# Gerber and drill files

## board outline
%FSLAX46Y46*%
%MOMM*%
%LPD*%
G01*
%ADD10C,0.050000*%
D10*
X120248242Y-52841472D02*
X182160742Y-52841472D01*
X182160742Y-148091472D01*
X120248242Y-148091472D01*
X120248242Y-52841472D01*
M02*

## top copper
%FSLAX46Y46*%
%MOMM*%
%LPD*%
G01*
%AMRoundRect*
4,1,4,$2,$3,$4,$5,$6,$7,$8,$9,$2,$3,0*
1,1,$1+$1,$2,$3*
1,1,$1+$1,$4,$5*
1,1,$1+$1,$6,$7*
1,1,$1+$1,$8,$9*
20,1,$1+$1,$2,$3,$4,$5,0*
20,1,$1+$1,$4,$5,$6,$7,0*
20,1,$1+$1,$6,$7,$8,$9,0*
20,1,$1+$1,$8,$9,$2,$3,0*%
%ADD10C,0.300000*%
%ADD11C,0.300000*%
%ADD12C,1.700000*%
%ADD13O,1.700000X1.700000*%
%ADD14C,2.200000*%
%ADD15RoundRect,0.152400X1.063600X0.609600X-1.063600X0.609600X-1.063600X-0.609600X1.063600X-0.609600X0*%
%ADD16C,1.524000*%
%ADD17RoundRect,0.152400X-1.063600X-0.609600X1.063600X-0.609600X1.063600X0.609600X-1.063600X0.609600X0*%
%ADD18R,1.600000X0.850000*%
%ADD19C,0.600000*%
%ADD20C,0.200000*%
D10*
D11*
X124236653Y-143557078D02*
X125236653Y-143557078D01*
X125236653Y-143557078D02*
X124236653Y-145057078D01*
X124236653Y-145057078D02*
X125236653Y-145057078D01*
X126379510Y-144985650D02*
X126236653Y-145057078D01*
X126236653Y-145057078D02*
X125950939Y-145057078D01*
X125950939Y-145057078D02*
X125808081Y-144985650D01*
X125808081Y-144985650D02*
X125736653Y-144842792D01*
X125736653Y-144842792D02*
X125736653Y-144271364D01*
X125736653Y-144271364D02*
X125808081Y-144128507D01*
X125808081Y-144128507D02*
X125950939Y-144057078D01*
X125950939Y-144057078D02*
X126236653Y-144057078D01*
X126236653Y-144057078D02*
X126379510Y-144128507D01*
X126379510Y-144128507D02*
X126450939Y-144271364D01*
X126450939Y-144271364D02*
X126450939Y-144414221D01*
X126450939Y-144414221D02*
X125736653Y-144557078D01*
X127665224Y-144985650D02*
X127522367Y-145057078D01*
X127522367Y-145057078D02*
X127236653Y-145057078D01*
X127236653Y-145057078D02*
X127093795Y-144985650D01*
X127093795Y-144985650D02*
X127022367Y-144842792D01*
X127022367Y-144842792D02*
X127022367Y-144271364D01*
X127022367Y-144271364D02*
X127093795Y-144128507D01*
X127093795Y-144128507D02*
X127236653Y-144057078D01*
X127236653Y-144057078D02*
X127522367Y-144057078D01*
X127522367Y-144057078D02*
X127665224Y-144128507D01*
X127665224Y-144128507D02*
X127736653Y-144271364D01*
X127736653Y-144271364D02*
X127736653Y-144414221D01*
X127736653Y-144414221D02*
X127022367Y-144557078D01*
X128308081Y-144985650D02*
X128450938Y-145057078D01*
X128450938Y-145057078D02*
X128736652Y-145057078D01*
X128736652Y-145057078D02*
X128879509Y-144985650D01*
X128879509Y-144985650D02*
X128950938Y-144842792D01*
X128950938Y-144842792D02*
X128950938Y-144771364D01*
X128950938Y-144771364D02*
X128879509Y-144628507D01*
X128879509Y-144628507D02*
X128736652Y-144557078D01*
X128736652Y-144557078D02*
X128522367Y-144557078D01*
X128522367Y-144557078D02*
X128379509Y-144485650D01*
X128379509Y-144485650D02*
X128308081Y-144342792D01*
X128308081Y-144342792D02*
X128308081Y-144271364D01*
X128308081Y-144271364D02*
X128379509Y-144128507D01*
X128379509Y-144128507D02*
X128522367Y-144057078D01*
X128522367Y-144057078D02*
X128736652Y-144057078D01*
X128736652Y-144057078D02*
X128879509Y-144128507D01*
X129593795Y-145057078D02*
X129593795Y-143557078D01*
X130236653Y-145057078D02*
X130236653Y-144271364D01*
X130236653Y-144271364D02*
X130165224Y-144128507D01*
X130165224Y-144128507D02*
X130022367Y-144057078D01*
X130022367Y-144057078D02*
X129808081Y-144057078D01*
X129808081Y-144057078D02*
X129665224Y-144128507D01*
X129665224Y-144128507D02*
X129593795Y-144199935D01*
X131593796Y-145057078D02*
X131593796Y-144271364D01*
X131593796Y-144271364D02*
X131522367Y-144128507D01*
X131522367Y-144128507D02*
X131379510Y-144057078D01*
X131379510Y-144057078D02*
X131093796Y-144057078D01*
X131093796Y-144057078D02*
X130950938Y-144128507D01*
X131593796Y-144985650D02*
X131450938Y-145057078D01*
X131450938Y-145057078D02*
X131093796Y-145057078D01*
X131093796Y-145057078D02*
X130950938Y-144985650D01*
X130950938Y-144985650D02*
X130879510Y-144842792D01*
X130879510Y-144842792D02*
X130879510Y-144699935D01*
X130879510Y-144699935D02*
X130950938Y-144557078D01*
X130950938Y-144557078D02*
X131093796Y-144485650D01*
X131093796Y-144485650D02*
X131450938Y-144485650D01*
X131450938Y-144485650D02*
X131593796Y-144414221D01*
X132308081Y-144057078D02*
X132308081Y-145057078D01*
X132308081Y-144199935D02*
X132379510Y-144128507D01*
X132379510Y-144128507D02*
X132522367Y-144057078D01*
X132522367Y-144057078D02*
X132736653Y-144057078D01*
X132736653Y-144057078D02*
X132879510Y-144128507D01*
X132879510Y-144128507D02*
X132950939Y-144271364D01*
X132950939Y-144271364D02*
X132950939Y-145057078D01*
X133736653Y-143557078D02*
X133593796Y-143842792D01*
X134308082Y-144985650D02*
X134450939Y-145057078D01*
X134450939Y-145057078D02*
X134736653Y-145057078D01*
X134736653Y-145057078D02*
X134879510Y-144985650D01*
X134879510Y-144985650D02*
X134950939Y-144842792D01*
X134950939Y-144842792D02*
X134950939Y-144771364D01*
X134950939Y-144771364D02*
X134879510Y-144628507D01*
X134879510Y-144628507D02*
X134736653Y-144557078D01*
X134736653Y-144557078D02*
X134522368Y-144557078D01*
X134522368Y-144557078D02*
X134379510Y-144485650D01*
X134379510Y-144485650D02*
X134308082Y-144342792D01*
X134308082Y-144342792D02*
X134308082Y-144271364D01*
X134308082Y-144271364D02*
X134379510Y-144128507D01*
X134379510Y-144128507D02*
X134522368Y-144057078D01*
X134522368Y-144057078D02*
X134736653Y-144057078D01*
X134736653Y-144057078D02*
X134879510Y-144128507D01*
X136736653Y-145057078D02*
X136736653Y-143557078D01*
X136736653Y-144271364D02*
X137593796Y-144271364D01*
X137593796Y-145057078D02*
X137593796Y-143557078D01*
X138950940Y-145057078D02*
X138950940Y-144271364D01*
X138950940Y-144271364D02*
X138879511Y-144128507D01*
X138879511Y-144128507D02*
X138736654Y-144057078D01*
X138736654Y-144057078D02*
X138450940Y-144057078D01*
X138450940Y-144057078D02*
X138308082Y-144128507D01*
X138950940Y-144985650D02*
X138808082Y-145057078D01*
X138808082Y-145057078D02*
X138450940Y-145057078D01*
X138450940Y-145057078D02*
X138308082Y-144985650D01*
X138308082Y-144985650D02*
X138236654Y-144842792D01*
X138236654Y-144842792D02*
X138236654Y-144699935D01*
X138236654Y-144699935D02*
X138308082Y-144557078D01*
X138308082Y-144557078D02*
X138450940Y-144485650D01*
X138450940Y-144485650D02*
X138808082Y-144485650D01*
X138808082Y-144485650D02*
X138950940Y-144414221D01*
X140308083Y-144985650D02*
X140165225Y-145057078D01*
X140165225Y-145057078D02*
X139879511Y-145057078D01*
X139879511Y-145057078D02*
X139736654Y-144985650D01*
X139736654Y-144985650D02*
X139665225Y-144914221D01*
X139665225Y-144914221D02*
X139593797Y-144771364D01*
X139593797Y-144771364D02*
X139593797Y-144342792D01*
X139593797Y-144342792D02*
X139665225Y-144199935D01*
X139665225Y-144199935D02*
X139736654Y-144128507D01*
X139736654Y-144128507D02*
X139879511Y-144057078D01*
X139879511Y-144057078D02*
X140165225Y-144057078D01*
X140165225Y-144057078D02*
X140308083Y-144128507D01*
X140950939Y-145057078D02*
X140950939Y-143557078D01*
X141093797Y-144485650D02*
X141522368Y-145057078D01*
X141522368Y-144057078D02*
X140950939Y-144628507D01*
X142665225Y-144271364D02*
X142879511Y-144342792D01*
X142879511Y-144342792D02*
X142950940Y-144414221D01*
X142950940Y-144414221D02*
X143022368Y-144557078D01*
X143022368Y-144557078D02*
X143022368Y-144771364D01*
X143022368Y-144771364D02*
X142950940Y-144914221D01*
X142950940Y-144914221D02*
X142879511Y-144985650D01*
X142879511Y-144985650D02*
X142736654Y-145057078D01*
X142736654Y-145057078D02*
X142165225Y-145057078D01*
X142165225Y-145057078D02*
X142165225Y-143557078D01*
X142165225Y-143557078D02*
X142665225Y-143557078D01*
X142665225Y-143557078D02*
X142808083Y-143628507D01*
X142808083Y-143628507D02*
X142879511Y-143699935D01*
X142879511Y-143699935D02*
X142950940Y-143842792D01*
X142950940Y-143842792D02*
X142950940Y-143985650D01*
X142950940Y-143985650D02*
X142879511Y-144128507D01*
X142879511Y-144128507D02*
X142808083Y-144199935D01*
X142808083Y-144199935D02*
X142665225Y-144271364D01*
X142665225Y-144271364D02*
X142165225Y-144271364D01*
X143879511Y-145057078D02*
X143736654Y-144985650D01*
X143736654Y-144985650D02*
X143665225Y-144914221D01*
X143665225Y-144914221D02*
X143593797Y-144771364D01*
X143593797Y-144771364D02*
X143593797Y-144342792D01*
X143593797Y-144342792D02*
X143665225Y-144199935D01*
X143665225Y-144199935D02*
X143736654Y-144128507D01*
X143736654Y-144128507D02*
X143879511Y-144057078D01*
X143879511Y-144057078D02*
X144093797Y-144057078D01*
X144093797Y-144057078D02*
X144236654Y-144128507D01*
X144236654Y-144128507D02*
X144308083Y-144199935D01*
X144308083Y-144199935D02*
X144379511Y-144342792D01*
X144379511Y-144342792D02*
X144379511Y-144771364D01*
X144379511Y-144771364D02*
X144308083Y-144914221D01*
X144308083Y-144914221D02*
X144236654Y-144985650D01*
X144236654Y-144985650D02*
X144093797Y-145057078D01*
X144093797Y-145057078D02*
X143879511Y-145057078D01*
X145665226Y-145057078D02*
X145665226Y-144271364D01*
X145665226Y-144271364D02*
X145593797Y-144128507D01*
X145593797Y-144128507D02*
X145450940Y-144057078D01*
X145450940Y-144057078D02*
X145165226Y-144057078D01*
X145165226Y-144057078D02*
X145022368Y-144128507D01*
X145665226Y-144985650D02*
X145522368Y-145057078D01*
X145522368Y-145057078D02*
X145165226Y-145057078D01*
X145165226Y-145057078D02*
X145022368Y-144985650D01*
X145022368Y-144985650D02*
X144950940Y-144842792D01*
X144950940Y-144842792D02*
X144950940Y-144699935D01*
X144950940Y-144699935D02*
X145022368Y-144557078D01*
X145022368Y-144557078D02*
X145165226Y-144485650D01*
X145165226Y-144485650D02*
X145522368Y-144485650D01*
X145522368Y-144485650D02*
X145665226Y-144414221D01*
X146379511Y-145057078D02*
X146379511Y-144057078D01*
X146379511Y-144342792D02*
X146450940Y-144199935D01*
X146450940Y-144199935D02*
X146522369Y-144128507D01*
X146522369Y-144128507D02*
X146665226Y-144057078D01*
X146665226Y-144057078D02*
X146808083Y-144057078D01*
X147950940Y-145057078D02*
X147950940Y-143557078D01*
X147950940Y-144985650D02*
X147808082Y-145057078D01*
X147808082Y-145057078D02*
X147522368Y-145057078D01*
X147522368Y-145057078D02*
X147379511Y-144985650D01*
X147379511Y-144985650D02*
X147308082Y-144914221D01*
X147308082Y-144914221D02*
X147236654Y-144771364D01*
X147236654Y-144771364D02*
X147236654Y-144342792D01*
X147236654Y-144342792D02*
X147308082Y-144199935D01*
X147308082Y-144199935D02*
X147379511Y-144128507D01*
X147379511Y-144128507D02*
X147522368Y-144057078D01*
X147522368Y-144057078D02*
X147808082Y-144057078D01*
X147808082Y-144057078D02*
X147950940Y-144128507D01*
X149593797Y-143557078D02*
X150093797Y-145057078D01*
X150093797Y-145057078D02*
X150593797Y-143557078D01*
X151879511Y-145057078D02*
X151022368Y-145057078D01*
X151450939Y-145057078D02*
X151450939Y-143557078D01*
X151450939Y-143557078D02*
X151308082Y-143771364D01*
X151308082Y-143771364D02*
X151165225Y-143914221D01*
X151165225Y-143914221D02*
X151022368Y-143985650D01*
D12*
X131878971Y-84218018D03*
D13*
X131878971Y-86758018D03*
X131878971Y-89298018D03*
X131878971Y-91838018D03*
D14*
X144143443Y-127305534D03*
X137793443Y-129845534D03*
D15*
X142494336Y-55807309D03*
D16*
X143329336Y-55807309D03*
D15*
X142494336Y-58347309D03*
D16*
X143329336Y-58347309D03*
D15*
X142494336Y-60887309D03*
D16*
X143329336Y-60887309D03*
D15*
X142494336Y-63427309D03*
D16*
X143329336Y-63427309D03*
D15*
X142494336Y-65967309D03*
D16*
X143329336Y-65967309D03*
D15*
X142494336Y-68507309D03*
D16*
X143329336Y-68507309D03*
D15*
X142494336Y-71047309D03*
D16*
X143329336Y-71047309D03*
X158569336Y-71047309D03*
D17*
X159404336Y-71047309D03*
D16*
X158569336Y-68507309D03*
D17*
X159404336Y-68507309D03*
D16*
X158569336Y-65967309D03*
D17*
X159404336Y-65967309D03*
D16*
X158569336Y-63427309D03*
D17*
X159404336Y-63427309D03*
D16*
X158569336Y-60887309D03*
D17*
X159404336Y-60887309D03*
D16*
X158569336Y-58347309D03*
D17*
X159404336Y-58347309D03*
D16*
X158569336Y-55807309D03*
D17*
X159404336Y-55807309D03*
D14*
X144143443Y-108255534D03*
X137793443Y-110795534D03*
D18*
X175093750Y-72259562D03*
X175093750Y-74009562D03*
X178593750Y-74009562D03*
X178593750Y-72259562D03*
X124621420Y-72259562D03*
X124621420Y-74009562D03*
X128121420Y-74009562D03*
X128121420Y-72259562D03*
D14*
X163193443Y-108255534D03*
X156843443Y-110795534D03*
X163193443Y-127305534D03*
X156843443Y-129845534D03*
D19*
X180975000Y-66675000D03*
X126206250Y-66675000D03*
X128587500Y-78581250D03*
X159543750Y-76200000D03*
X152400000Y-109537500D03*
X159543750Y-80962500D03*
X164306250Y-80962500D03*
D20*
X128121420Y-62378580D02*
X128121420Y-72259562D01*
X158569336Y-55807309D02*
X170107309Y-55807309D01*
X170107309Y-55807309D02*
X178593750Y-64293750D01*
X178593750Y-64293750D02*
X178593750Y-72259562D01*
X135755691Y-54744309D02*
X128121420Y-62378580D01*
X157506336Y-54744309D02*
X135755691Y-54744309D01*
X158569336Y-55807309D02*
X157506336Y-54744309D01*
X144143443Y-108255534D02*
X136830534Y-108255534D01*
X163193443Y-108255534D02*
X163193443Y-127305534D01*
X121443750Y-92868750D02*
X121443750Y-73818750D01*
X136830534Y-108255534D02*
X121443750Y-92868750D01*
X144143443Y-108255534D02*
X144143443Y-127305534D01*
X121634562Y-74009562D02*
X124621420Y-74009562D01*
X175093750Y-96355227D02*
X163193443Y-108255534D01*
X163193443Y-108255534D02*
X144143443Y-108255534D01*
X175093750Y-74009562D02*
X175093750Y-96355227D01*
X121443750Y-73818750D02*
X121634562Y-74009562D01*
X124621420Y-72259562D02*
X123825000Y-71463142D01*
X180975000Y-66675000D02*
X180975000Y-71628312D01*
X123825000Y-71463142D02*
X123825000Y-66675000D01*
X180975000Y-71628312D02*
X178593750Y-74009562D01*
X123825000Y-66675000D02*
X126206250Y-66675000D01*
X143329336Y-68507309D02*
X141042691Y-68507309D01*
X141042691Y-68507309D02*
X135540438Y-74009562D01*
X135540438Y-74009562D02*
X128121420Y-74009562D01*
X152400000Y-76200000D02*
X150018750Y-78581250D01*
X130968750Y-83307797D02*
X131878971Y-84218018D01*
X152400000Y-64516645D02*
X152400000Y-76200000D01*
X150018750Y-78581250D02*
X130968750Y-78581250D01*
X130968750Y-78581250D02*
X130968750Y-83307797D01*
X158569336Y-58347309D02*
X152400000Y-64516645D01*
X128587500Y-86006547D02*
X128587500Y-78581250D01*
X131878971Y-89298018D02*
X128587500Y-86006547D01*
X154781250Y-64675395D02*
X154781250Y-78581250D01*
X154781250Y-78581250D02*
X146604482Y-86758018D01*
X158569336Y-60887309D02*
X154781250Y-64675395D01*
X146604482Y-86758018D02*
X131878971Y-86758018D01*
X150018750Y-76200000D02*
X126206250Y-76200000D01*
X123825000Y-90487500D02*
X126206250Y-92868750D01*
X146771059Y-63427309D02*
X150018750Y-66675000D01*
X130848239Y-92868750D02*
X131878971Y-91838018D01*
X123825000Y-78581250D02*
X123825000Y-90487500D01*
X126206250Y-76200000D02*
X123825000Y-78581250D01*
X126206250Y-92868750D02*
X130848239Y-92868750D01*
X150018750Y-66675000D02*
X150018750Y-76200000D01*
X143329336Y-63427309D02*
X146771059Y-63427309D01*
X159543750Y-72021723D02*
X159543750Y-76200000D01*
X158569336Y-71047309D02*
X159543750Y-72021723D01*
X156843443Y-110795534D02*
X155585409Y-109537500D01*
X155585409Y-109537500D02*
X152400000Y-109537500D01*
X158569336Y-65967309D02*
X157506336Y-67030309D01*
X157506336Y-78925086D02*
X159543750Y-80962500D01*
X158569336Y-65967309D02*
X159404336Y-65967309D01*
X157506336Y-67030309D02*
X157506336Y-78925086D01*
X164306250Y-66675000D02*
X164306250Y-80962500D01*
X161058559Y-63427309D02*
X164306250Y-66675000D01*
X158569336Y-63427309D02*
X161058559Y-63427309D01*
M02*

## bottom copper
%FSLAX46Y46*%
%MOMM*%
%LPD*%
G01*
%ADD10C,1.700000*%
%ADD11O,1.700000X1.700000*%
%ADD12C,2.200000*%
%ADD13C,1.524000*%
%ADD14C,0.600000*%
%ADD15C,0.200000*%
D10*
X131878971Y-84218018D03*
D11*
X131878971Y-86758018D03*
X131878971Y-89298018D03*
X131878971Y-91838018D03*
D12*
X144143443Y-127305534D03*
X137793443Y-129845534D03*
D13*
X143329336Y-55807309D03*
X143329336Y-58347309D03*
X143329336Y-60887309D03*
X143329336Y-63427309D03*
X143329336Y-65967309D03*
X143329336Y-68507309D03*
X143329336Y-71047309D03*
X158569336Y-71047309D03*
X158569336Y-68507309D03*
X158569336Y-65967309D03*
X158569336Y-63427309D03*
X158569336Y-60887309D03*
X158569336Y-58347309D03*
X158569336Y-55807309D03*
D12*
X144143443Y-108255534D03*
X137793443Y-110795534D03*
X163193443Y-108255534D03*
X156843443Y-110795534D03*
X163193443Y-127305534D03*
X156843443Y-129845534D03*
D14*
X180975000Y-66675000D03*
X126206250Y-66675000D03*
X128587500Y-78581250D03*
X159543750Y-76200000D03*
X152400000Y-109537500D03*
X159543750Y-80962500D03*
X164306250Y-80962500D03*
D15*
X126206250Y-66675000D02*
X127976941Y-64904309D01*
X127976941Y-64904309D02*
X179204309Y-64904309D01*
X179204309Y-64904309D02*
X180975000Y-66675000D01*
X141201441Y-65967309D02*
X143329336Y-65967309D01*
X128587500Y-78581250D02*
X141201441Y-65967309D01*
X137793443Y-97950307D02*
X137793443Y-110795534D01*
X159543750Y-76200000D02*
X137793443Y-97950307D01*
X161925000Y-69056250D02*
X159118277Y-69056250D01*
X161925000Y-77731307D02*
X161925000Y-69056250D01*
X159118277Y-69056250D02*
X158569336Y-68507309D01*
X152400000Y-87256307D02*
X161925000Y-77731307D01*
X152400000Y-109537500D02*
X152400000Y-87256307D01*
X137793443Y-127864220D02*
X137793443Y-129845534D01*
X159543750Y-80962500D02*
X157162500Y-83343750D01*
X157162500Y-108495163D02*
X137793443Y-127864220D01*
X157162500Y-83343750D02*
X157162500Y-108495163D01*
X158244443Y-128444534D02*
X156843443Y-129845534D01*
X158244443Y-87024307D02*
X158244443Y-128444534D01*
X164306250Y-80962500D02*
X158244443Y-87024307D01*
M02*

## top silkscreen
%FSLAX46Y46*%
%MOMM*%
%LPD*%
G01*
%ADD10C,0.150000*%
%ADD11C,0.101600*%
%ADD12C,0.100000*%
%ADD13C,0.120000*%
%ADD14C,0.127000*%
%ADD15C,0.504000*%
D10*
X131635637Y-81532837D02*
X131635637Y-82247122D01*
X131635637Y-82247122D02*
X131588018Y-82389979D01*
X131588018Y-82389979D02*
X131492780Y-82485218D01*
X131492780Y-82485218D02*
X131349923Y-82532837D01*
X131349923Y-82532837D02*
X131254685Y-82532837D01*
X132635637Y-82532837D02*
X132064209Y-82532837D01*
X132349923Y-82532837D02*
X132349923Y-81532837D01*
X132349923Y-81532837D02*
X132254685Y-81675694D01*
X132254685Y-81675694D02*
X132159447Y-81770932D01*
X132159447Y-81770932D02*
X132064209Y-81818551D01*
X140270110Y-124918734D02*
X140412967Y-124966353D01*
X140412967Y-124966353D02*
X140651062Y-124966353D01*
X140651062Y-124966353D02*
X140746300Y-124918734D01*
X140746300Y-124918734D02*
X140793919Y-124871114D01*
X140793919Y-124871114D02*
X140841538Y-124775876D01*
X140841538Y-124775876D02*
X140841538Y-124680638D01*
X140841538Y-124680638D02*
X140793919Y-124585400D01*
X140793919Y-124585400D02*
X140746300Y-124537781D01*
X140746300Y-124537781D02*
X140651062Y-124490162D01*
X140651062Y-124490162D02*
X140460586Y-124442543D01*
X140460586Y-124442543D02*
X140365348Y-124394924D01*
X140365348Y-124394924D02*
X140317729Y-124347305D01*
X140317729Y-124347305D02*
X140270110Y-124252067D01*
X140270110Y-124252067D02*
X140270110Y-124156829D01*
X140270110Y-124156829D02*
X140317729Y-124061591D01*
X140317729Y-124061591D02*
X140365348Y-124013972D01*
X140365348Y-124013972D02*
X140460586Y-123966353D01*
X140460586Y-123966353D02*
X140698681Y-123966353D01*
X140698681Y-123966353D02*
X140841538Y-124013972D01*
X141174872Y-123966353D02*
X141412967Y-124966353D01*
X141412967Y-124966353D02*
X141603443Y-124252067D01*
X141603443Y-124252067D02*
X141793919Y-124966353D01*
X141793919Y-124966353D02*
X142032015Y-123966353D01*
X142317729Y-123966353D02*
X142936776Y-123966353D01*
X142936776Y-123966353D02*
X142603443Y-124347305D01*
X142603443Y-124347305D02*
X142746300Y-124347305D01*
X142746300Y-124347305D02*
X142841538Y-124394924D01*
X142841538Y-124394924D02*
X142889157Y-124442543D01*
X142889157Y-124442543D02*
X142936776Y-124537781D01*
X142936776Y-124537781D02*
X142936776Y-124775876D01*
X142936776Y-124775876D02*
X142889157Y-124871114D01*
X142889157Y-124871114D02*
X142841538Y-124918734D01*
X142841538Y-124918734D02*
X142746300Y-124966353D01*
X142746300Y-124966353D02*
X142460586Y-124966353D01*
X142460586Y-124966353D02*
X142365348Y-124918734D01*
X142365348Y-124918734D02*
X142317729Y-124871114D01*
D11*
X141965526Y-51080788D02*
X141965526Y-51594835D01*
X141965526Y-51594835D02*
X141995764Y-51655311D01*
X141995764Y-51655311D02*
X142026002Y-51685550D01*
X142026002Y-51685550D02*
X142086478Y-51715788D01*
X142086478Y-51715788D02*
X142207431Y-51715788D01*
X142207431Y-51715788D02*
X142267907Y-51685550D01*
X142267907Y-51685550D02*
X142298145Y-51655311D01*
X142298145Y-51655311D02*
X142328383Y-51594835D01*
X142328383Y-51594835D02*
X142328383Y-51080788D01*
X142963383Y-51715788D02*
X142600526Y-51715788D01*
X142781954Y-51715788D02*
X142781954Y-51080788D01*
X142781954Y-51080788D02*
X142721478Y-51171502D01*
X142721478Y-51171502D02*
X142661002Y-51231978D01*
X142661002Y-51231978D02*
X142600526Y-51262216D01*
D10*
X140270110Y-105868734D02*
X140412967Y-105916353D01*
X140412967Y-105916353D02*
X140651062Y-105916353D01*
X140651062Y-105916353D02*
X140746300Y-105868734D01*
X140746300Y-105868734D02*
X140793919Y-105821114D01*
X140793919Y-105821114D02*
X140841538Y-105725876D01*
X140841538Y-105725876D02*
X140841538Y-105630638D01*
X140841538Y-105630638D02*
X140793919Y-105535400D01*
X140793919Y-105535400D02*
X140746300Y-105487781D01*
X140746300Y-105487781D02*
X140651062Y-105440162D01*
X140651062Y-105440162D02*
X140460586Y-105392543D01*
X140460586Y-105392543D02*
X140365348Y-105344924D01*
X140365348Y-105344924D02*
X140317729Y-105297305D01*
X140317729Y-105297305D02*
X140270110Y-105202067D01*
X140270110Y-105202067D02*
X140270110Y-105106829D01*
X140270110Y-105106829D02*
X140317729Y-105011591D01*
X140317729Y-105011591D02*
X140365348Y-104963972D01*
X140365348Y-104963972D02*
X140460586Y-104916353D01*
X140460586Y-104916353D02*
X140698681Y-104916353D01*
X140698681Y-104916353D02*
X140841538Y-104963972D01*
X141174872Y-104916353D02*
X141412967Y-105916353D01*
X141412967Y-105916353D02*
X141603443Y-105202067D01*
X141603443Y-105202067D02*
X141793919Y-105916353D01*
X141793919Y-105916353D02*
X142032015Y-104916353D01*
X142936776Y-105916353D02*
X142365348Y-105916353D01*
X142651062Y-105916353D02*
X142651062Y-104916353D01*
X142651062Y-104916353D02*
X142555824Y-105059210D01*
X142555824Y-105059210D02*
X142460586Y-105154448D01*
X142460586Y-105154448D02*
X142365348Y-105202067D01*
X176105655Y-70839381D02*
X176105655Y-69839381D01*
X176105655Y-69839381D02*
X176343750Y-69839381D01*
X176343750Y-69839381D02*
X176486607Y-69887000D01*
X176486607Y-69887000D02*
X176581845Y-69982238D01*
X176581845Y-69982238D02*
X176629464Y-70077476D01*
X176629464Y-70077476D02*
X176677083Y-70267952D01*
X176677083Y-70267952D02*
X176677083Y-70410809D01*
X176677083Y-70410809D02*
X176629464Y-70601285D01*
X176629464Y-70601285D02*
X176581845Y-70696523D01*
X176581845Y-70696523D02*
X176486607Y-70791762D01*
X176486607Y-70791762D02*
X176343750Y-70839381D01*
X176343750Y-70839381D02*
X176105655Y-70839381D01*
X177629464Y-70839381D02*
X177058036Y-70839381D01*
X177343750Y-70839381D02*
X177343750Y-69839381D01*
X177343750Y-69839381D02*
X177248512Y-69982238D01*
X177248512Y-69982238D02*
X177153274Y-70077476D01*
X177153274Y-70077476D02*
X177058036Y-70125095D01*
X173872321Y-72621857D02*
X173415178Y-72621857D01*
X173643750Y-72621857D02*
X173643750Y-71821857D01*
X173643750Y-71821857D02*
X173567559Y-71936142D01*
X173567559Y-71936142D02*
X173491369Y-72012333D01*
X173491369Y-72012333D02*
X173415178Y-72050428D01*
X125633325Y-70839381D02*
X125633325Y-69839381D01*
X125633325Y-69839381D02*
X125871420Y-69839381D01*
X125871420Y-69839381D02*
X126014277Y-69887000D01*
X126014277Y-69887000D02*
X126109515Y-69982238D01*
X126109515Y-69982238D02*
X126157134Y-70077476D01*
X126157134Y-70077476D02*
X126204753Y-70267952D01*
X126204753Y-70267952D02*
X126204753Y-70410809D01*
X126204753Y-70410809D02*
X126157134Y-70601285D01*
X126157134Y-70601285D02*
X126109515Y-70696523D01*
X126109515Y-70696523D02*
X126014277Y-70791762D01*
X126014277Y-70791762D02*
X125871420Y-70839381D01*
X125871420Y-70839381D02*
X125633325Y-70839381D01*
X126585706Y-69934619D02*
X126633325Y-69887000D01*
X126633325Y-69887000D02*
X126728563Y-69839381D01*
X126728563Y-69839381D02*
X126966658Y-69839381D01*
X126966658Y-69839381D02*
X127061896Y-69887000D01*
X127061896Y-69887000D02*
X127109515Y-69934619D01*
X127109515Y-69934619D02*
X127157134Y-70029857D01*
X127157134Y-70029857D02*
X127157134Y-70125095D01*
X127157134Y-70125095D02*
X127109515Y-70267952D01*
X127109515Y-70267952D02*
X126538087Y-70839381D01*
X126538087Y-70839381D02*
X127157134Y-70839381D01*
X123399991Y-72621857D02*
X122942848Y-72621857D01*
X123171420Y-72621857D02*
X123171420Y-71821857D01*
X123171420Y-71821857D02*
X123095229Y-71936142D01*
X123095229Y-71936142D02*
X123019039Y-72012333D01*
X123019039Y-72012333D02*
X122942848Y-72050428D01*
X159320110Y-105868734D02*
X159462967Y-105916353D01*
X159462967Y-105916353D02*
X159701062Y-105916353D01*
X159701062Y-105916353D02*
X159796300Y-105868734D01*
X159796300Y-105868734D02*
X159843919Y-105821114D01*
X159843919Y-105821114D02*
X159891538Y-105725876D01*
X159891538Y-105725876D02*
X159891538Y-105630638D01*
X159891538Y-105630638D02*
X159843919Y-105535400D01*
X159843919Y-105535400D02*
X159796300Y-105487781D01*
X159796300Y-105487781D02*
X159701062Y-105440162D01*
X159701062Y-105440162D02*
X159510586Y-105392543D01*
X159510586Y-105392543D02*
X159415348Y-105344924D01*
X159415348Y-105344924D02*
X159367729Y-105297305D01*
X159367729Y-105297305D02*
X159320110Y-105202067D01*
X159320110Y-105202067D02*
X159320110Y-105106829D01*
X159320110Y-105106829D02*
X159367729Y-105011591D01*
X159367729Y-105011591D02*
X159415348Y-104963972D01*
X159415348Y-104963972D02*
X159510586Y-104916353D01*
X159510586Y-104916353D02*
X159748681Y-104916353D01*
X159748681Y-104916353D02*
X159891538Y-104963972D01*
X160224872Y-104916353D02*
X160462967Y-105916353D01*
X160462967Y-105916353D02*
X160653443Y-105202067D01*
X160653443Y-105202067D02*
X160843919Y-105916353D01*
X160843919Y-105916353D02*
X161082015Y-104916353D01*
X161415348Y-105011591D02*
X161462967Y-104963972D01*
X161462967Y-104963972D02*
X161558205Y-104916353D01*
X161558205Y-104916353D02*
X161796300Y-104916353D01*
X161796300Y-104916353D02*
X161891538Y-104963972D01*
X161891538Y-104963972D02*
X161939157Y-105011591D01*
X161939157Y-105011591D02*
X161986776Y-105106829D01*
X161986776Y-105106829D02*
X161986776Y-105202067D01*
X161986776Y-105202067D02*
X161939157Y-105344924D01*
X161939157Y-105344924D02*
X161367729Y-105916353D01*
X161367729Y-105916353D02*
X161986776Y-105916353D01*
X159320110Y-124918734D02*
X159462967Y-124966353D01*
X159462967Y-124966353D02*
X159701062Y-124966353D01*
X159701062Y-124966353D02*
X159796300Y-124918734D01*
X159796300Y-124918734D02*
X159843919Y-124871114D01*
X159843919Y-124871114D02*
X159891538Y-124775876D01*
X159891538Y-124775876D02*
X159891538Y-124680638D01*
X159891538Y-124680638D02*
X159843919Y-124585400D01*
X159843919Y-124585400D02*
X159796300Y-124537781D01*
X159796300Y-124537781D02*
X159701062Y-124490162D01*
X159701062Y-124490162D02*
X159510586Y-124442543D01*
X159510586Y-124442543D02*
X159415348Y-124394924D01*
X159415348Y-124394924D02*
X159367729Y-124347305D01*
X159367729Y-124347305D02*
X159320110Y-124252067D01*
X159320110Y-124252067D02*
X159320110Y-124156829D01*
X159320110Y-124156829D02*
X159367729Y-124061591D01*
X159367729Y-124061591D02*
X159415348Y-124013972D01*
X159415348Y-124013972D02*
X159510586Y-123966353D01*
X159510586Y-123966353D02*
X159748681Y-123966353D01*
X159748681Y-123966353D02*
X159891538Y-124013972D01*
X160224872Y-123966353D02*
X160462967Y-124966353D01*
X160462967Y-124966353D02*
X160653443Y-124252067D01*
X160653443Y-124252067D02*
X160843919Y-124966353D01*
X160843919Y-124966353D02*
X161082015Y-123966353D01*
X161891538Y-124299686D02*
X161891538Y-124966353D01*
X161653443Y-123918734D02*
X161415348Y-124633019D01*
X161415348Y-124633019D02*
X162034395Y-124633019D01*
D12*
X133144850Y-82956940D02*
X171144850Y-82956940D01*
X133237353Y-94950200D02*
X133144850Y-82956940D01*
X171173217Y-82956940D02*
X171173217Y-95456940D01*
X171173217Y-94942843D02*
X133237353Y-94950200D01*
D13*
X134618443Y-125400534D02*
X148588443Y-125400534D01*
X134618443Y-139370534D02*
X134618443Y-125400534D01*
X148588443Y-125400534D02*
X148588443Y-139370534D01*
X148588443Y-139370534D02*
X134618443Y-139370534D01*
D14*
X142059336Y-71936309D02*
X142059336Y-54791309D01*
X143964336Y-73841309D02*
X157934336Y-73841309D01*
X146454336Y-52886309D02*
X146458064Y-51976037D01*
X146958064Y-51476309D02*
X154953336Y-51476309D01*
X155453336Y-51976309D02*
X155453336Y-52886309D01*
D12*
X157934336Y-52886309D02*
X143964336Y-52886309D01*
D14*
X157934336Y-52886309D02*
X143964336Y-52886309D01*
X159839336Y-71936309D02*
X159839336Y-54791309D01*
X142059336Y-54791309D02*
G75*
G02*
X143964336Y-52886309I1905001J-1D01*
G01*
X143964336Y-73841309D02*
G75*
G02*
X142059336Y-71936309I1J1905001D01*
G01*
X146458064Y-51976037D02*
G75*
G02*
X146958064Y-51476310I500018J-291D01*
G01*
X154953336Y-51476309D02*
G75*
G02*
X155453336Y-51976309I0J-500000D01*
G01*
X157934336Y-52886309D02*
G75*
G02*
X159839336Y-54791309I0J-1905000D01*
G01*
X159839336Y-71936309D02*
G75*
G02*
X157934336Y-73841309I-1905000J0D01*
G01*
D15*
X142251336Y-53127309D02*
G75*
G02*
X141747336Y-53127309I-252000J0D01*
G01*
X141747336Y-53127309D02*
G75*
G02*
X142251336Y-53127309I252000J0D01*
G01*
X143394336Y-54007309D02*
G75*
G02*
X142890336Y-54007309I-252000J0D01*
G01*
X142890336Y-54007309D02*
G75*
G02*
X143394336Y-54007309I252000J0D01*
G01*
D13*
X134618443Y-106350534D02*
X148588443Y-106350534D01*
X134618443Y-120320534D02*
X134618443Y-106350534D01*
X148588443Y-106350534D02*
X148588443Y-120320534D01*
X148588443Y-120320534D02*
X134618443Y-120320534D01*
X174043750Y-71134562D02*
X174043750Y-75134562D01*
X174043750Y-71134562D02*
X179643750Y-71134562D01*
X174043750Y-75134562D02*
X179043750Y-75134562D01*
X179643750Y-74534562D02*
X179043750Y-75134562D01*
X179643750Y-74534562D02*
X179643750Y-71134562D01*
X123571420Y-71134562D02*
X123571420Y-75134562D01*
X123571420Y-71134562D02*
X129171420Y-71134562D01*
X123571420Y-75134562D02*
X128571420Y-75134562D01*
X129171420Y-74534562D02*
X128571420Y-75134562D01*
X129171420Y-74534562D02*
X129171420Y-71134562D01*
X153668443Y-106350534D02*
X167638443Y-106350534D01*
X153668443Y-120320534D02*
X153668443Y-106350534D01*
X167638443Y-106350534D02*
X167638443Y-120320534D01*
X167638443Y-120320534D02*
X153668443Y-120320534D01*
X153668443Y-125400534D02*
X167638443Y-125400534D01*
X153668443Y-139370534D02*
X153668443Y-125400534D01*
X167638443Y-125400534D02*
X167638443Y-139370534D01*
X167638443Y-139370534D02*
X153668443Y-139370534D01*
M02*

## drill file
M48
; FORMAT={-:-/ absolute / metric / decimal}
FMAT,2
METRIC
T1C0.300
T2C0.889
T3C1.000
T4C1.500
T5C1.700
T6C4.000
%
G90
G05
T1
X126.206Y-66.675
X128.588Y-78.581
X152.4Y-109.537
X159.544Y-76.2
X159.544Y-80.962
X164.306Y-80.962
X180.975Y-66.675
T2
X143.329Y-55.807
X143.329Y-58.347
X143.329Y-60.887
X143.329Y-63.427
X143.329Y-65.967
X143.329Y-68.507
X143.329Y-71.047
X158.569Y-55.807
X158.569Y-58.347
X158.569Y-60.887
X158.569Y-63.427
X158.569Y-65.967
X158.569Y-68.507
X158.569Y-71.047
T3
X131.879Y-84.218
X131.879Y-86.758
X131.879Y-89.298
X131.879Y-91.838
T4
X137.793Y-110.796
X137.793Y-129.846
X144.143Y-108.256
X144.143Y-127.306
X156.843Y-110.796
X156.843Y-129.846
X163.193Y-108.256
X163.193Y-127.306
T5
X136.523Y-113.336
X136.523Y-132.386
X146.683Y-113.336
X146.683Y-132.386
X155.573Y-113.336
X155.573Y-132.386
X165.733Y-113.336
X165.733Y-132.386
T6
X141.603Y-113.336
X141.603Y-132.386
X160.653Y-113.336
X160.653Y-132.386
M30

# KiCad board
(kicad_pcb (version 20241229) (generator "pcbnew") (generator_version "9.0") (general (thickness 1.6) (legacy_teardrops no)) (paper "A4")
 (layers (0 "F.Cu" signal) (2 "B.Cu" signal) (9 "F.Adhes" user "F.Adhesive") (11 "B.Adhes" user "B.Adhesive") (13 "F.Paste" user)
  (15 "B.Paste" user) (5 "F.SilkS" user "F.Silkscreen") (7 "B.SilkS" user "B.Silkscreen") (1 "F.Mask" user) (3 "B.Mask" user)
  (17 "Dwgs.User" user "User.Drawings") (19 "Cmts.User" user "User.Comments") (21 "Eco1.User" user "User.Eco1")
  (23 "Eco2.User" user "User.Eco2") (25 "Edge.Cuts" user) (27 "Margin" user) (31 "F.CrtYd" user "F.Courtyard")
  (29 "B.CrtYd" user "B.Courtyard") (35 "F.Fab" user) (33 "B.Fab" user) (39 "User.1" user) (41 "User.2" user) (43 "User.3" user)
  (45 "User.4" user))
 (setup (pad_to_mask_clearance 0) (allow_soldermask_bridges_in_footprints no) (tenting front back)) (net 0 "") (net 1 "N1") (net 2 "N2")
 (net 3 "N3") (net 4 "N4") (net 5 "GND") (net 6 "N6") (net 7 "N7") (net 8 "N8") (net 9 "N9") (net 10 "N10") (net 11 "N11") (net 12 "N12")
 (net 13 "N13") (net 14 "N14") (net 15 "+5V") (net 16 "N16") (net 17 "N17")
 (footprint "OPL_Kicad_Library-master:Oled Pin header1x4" (layer "F.Cu") (at 131.878971 84.218018)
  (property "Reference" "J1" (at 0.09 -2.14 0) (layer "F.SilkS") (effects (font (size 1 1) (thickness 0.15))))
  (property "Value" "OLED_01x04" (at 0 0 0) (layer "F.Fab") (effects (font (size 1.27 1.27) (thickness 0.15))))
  (fp_line (start 1.265879 -1.261078) (end 39.265879 -1.261078) (stroke (width 0.1) (type solid)) (layer "F.SilkS"))
  (fp_line (start 1.358382 10.732182) (end 1.265879 -1.261078) (stroke (width 0.1) (type default)) (layer "F.SilkS"))
  (fp_line (start 39.294246 -1.261078) (end 39.294246 11.238922) (stroke (width 0.1) (type solid)) (layer "F.SilkS"))
  (fp_line (start 39.294246 10.724825) (end 1.358382 10.732182) (stroke (width 0.1) (type default)) (layer "F.SilkS"))
  (pad "1" thru_hole circle (at 0 0) (size 1.7 1.7) (drill 1) (layers "*.Cu" "*.Mask") (remove_unused_layers no) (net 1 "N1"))
  (pad "2" thru_hole oval (at 0 2.54) (size 1.7 1.7) (drill 1) (layers "*.Cu" "*.Mask") (remove_unused_layers no) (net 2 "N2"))
  (pad "3" thru_hole oval (at 0 5.08) (size 1.7 1.7) (drill 1) (layers "*.Cu" "*.Mask") (remove_unused_layers no) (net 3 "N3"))
  (pad "4" thru_hole oval (at 0 7.62) (size 1.7 1.7) (drill 1) (layers "*.Cu" "*.Mask") (remove_unused_layers no) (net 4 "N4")))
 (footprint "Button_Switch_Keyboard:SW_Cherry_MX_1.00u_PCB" (layer "F.Cu") (at 144.143443 127.305534)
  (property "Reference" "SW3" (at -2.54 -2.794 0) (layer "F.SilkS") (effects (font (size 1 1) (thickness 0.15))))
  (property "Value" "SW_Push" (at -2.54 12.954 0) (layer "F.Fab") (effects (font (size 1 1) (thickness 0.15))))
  (fp_line (start -9.525 -1.905) (end 4.445 -1.905) (stroke (width 0.12) (type solid)) (layer "F.SilkS"))
  (fp_line (start -9.525 12.065) (end -9.525 -1.905) (stroke (width 0.12) (type solid)) (layer "F.SilkS"))
  (fp_line (start 4.445 -1.905) (end 4.445 12.065) (stroke (width 0.12) (type solid)) (layer "F.SilkS"))
  (fp_line (start 4.445 12.065) (end -9.525 12.065) (stroke (width 0.12) (type solid)) (layer "F.SilkS"))
  (pad "" np_thru_hole circle (at -7.62 5.08) (size 1.7 1.7) (drill 1.7) (layers "*.Cu" "*.Mask"))
  (pad "" np_thru_hole circle (at -2.54 5.08) (size 4 4) (drill 4) (layers "*.Cu" "*.Mask"))
  (pad "" np_thru_hole circle (at 2.54 5.08) (size 1.7 1.7) (drill 1.7) (layers "*.Cu" "*.Mask"))
  (pad "1" thru_hole circle (at 0 0) (size 2.2 2.2) (drill 1.5) (layers "*.Cu" "*.Mask") (remove_unused_layers no) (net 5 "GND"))
  (pad "2" thru_hole circle (at -6.35 2.54) (size 2.2 2.2) (drill 1.5) (layers "*.Cu" "*.Mask") (remove_unused_layers no) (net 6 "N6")))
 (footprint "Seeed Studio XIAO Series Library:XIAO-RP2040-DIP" (layer "F.Cu") (at 150.949336 63.427309)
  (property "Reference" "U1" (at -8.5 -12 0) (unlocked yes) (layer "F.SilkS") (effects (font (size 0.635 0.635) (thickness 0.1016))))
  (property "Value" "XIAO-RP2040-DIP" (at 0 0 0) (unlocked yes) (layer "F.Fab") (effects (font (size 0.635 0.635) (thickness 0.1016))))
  (fp_line (start -8.89 8.509) (end -8.89 -8.636) (stroke (width 0.127) (type solid)) (layer "F.SilkS"))
  (fp_line (start -6.985 10.414) (end 6.985 10.414) (stroke (width 0.127) (type solid)) (layer "F.SilkS"))
  (fp_line (start -4.495 -10.541) (end -4.491272 -11.451272) (stroke (width 0.127) (type solid)) (layer "F.SilkS"))
  (fp_line (start -3.991272 -11.951) (end 4.004 -11.951) (stroke (width 0.127) (type solid)) (layer "F.SilkS"))
  (fp_line (start 4.504 -11.451) (end 4.504 -10.541) (stroke (width 0.127) (type solid)) (layer "F.SilkS"))
  (fp_line (start 6.985 -10.541) (end -6.985 -10.541) (stroke (width 0.1) (type solid)) (layer "F.SilkS"))
  (fp_line (start 6.985 -10.541) (end -6.985 -10.541) (stroke (width 0.127) (type solid)) (layer "F.SilkS"))
  (fp_line (start 8.89 8.509) (end 8.89 -8.636) (stroke (width 0.127) (type solid)) (layer "F.SilkS"))
  (fp_arc (start -8.89 -8.636) (mid -8.332038 -9.983038) (end -6.985 -10.541) (stroke (width 0.127) (type solid)) (layer "F.SilkS"))
  (fp_arc (start -6.985 10.414) (mid -8.332038 9.856038) (end -8.89 8.509) (stroke (width 0.127) (type solid)) (layer "F.SilkS"))
  (fp_arc (start -4.491272 -11.451272) (mid -4.344728 -11.80464) (end -3.991272 -11.951) (stroke (width 0.127) (type default))
   (layer "F.SilkS"))
  (fp_arc (start 4.004 -11.951) (mid 4.357553 -11.804553) (end 4.504 -11.451) (stroke (width 0.127) (type default)) (layer "F.SilkS"))
  (fp_arc (start 6.985 -10.541) (mid 8.332038 -9.983038) (end 8.89 -8.636) (stroke (width 0.127) (type solid)) (layer "F.SilkS"))
  (fp_arc (start 8.89 8.509) (mid 8.332038 9.856038) (end 6.985 10.414) (stroke (width 0.127) (type solid)) (layer "F.SilkS"))
  (fp_circle (center -8.95 -10.3) (end -8.95 -10.554) (stroke (width 0.5) (type solid)) (fill yes) (layer "F.SilkS"))
  (fp_circle (center -7.807 -9.42) (end -7.807 -9.674) (stroke (width 0.5) (type solid)) (fill yes) (layer "F.SilkS"))
  (pad "1" smd roundrect (at -8.455 -7.62 180) (size 2.432 1.524) (layers "F.Cu" "F.Mask") (roundrect_rratio 0.1) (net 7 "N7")
   (thermal_bridge_angle 45))
  (pad "1" thru_hole circle (at -7.62 -7.62 180) (size 1.524 1.524) (drill 0.889) (layers "*.Cu" "*.Mask") (remove_unused_layers no)
   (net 7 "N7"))
  (pad "2" smd roundrect (at -8.455 -5.08 180) (size 2.432 1.524) (layers "F.Cu" "F.Mask") (roundrect_rratio 0.1) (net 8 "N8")
   (thermal_bridge_angle 45))
  (pad "2" thru_hole circle (at -7.62 -5.08 180) (size 1.524 1.524) (drill 0.889) (layers "*.Cu" "*.Mask") (remove_unused_layers no)
   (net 8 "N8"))
  (pad "3" smd roundrect (at -8.455 -2.54 180) (size 2.432 1.524) (layers "F.Cu" "F.Mask") (roundrect_rratio 0.1) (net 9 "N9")
   (thermal_bridge_angle 45))
  (pad "3" thru_hole circle (at -7.62 -2.54 180) (size 1.524 1.524) (drill 0.889) (layers "*.Cu" "*.Mask") (remove_unused_layers no)
   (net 9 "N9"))
  (pad "4" smd roundrect (at -8.455 0 180) (size 2.432 1.524) (layers "F.Cu" "F.Mask") (roundrect_rratio 0.1) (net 4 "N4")
   (thermal_bridge_angle 45))
  (pad "4" thru_hole circle (at -7.62 0 180) (size 1.524 1.524) (drill 0.889) (layers "*.Cu" "*.Mask") (remove_unused_layers no)
   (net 4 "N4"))
  (pad "5" smd roundrect (at -8.455 2.54 180) (size 2.432 1.524) (layers "F.Cu" "F.Mask") (roundrect_rratio 0.1) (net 3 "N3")
   (thermal_bridge_angle 45))
  (pad "5" thru_hole circle (at -7.62 2.54 180) (size 1.524 1.524) (drill 0.889) (layers "*.Cu" "*.Mask") (remove_unused_layers no)
   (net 3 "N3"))
  (pad "6" smd roundrect (at -8.455 5.08 180) (size 2.432 1.524) (layers "F.Cu" "F.Mask") (roundrect_rratio 0.1) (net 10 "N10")
   (thermal_bridge_angle 45))
  (pad "6" thru_hole circle (at -7.62 5.08 180) (size 1.524 1.524) (drill 0.889) (layers "*.Cu" "*.Mask") (remove_unused_layers no)
   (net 10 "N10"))
  (pad "7" smd roundrect (at -8.455 7.62 180) (size 2.432 1.524) (layers "F.Cu" "F.Mask") (roundrect_rratio 0.1) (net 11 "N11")
   (thermal_bridge_angle 45))
  (pad "7" thru_hole circle (at -7.62 7.62 180) (size 1.524 1.524) (drill 0.889) (layers "*.Cu" "*.Mask") (remove_unused_layers no)
   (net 11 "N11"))
  (pad "8" thru_hole circle (at 7.62 7.62) (size 1.524 1.524) (drill 0.889) (layers "*.Cu" "*.Mask") (remove_unused_layers no)
   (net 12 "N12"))
  (pad "8" smd roundrect (at 8.455 7.62) (size 2.432 1.524) (layers "F.Cu" "F.Mask") (roundrect_rratio 0.1) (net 12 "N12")
   (thermal_bridge_angle 45))
  (pad "9" thru_hole circle (at 7.62 5.08) (size 1.524 1.524) (drill 0.889) (layers "*.Cu" "*.Mask") (remove_unused_layers no)
   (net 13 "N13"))
  (pad "9" smd roundrect (at 8.455 5.08) (size 2.432 1.524) (layers "F.Cu" "F.Mask") (roundrect_rratio 0.1) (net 13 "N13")
   (thermal_bridge_angle 45))
  (pad "10" thru_hole circle (at 7.62 2.54) (size 1.524 1.524) (drill 0.889) (layers "*.Cu" "*.Mask") (remove_unused_layers no) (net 6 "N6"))
  (pad "10" smd roundrect (at 8.455 2.54) (size 2.432 1.524) (layers "F.Cu" "F.Mask") (roundrect_rratio 0.1) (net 6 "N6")
   (thermal_bridge_angle 45))
  (pad "11" thru_hole circle (at 7.62 0) (size 1.524 1.524) (drill 0.889) (layers "*.Cu" "*.Mask") (remove_unused_layers no) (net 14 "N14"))
  (pad "11" smd roundrect (at 8.455 0) (size 2.432 1.524) (layers "F.Cu" "F.Mask") (roundrect_rratio 0.1) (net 14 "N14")
   (thermal_bridge_angle 45))
  (pad "12" thru_hole circle (at 7.62 -2.54) (size 1.524 1.524) (drill 0.889) (layers "*.Cu" "*.Mask") (remove_unused_layers no)
   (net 2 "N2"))
  (pad "12" smd roundrect (at 8.455 -2.54) (size 2.432 1.524) (layers "F.Cu" "F.Mask") (roundrect_rratio 0.1) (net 2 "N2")
   (thermal_bridge_angle 45))
  (pad "13" thru_hole circle (at 7.62 -5.08) (size 1.524 1.524) (drill 0.889) (layers "*.Cu" "*.Mask") (remove_unused_layers no)
   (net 1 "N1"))
  (pad "13" smd roundrect (at 8.455 -5.08) (size 2.432 1.524) (layers "F.Cu" "F.Mask") (roundrect_rratio 0.1) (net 1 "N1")
   (thermal_bridge_angle 45))
  (pad "14" thru_hole circle (at 7.62 -7.62) (size 1.524 1.524) (drill 0.889) (layers "*.Cu" "*.Mask") (remove_unused_layers no)
   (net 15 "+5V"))
  (pad "14" smd roundrect (at 8.455 -7.62) (size 2.432 1.524) (layers "F.Cu" "F.Mask") (roundrect_rratio 0.1) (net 15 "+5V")
   (thermal_bridge_angle 45)))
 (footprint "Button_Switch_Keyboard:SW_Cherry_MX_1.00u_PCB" (layer "F.Cu") (at 144.143443 108.255534)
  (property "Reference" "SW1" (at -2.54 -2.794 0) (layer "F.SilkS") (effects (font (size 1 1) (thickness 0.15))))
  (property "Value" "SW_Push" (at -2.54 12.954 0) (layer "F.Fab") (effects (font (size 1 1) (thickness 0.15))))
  (fp_line (start -9.525 -1.905) (end 4.445 -1.905) (stroke (width 0.12) (type solid)) (layer "F.SilkS"))
  (fp_line (start -9.525 12.065) (end -9.525 -1.905) (stroke (width 0.12) (type solid)) (layer "F.SilkS"))
  (fp_line (start 4.445 -1.905) (end 4.445 12.065) (stroke (width 0.12) (type solid)) (layer "F.SilkS"))
  (fp_line (start 4.445 12.065) (end -9.525 12.065) (stroke (width 0.12) (type solid)) (layer "F.SilkS"))
  (pad "" np_thru_hole circle (at -7.62 5.08) (size 1.7 1.7) (drill 1.7) (layers "*.Cu" "*.Mask"))
  (pad "" np_thru_hole circle (at -2.54 5.08) (size 4 4) (drill 4) (layers "*.Cu" "*.Mask"))
  (pad "" np_thru_hole circle (at 2.54 5.08) (size 1.7 1.7) (drill 1.7) (layers "*.Cu" "*.Mask"))
  (pad "1" thru_hole circle (at 0 0) (size 2.2 2.2) (drill 1.5) (layers "*.Cu" "*.Mask") (remove_unused_layers no) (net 5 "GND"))
  (pad "2" thru_hole circle (at -6.35 2.54) (size 2.2 2.2) (drill 1.5) (layers "*.Cu" "*.Mask") (remove_unused_layers no) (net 12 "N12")))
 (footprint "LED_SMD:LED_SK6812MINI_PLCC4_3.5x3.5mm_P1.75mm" (layer "F.Cu") (at 176.84375 73.134562)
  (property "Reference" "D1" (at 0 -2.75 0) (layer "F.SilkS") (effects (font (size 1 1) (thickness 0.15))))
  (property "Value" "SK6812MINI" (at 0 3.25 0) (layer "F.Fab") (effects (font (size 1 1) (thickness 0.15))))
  (fp_line (start -2.8 -2) (end -2.8 2) (stroke (width 0.12) (type default)) (layer "F.SilkS"))
  (fp_line (start -2.8 -2) (end 2.8 -2) (stroke (width 0.12) (type solid)) (layer "F.SilkS"))
  (fp_line (start -2.8 2) (end 2.2 2) (stroke (width 0.12) (type solid)) (layer "F.SilkS"))
  (fp_line (start 2.8 1.4) (end 2.2 2) (stroke (width 0.12) (type default)) (layer "F.SilkS"))
  (fp_line (start 2.8 1.4) (end 2.8 -2) (stroke (width 0.12) (type solid)) (layer "F.SilkS"))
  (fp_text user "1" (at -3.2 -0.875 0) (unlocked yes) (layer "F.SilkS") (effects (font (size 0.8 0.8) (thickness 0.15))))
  (pad "1" smd rect (at -1.75 -0.875) (size 1.6 0.85) (layers "F.Cu" "F.Mask" "F.Paste") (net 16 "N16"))
  (pad "2" smd rect (at -1.75 0.875) (size 1.6 0.85) (layers "F.Cu" "F.Mask" "F.Paste") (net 5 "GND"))
  (pad "3" smd rect (at 1.75 0.875) (size 1.6 0.85) (layers "F.Cu" "F.Mask" "F.Paste") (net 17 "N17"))
  (pad "4" smd rect (at 1.75 -0.875) (size 1.6 0.85) (layers "F.Cu" "F.Mask" "F.Paste") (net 15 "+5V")))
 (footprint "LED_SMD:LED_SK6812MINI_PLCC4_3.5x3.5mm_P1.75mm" (layer "F.Cu") (at 126.37142 73.134562)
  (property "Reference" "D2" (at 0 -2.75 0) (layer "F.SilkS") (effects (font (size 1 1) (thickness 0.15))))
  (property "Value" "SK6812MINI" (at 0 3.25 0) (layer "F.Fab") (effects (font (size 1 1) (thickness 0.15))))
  (fp_line (start -2.8 -2) (end -2.8 2) (stroke (width 0.12) (type default)) (layer "F.SilkS"))
  (fp_line (start -2.8 -2) (end 2.8 -2) (stroke (width 0.12) (type solid)) (layer "F.SilkS"))
  (fp_line (start -2.8 2) (end 2.2 2) (stroke (width 0.12) (type solid)) (layer "F.SilkS"))
  (fp_line (start 2.8 1.4) (end 2.2 2) (stroke (width 0.12) (type default)) (layer "F.SilkS"))
  (fp_line (start 2.8 1.4) (end 2.8 -2) (stroke (width 0.12) (type solid)) (layer "F.SilkS"))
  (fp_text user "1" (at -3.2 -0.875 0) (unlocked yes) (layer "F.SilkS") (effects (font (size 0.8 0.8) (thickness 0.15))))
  (pad "1" smd rect (at -1.75 -0.875) (size 1.6 0.85) (layers "F.Cu" "F.Mask" "F.Paste") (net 17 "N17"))
  (pad "2" smd rect (at -1.75 0.875) (size 1.6 0.85) (layers "F.Cu" "F.Mask" "F.Paste") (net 5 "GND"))
  (pad "3" smd rect (at 1.75 0.875) (size 1.6 0.85) (layers "F.Cu" "F.Mask" "F.Paste") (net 10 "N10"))
  (pad "4" smd rect (at 1.75 -0.875) (size 1.6 0.85) (layers "F.Cu" "F.Mask" "F.Paste") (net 15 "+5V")))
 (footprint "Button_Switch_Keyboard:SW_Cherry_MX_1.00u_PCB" (layer "F.Cu") (at 163.193443 108.255534)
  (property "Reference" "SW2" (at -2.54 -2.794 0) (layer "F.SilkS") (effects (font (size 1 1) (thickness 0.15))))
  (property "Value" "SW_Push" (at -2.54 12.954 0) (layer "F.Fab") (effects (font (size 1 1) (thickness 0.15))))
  (fp_line (start -9.525 -1.905) (end 4.445 -1.905) (stroke (width 0.12) (type solid)) (layer "F.SilkS"))
  (fp_line (start -9.525 12.065) (end -9.525 -1.905) (stroke (width 0.12) (type solid)) (layer "F.SilkS"))
  (fp_line (start 4.445 -1.905) (end 4.445 12.065) (stroke (width 0.12) (type solid)) (layer "F.SilkS"))
  (fp_line (start 4.445 12.065) (end -9.525 12.065) (stroke (width 0.12) (type solid)) (layer "F.SilkS"))
  (pad "" np_thru_hole circle (at -7.62 5.08) (size 1.7 1.7) (drill 1.7) (layers "*.Cu" "*.Mask"))
  (pad "" np_thru_hole circle (at -2.54 5.08) (size 4 4) (drill 4) (layers "*.Cu" "*.Mask"))
  (pad "" np_thru_hole circle (at 2.54 5.08) (size 1.7 1.7) (drill 1.7) (layers "*.Cu" "*.Mask"))
  (pad "1" thru_hole circle (at 0 0) (size 2.2 2.2) (drill 1.5) (layers "*.Cu" "*.Mask") (remove_unused_layers no) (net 5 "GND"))
  (pad "2" thru_hole circle (at -6.35 2.54) (size 2.2 2.2) (drill 1.5) (layers "*.Cu" "*.Mask") (remove_unused_layers no) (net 13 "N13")))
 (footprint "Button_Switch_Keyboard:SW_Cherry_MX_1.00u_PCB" (layer "F.Cu") (at 163.193443 127.305534)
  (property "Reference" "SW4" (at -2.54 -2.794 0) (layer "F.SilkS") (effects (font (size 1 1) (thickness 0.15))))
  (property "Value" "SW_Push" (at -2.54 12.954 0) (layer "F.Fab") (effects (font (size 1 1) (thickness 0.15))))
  (fp_line (start -9.525 -1.905) (end 4.445 -1.905) (stroke (width 0.12) (type solid)) (layer "F.SilkS"))
  (fp_line (start -9.525 12.065) (end -9.525 -1.905) (stroke (width 0.12) (type solid)) (layer "F.SilkS"))
  (fp_line (start 4.445 -1.905) (end 4.445 12.065) (stroke (width 0.12) (type solid)) (layer "F.SilkS"))
  (fp_line (start 4.445 12.065) (end -9.525 12.065) (stroke (width 0.12) (type solid)) (layer "F.SilkS"))
  (pad "" np_thru_hole circle (at -7.62 5.08) (size 1.7 1.7) (drill 1.7) (layers "*.Cu" "*.Mask"))
  (pad "" np_thru_hole circle (at -2.54 5.08) (size 4 4) (drill 4) (layers "*.Cu" "*.Mask"))
  (pad "" np_thru_hole circle (at 2.54 5.08) (size 1.7 1.7) (drill 1.7) (layers "*.Cu" "*.Mask"))
  (pad "1" thru_hole circle (at 0 0) (size 2.2 2.2) (drill 1.5) (layers "*.Cu" "*.Mask") (remove_unused_layers no) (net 5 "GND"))
  (pad "2" thru_hole circle (at -6.35 2.54) (size 2.2 2.2) (drill 1.5) (layers "*.Cu" "*.Mask") (remove_unused_layers no) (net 14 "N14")))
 (gr_rect (start 120.248242 52.841472) (end 182.160742 148.091472) (stroke (width 0.05) (type default)) (fill no) (layer "Edge.Cuts"))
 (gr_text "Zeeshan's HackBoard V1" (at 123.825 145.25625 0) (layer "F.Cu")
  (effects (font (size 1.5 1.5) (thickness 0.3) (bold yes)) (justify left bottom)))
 (segment (start 128.12142 62.37858) (end 128.12142 72.259562) (width 0.2) (layer "F.Cu") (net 15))
 (segment (start 158.569336 55.807309) (end 170.107309 55.807309) (width 0.2) (layer "F.Cu") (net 15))
 (segment (start 170.107309 55.807309) (end 178.59375 64.29375) (width 0.2) (layer "F.Cu") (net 15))
 (segment (start 178.59375 64.29375) (end 178.59375 72.259562) (width 0.2) (layer "F.Cu") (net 15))
 (segment (start 135.755691 54.744309) (end 128.12142 62.37858) (width 0.2) (layer "F.Cu") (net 15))
 (segment (start 157.506336 54.744309) (end 135.755691 54.744309) (width 0.2) (layer "F.Cu") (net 15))
 (segment (start 158.569336 55.807309) (end 157.506336 54.744309) (width 0.2) (layer "F.Cu") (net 15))
 (segment (start 144.143443 108.255534) (end 136.830534 108.255534) (width 0.2) (layer "F.Cu") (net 5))
 (segment (start 163.193443 108.255534) (end 163.193443 127.305534) (width 0.2) (layer "F.Cu") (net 5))
 (segment (start 121.44375 92.86875) (end 121.44375 73.81875) (width 0.2) (layer "F.Cu") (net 5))
 (segment (start 136.830534 108.255534) (end 121.44375 92.86875) (width 0.2) (layer "F.Cu") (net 5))
 (segment (start 144.143443 108.255534) (end 144.143443 127.305534) (width 0.2) (layer "F.Cu") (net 5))
 (segment (start 121.634562 74.009562) (end 124.62142 74.009562) (width 0.2) (layer "F.Cu") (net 5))
 (segment (start 175.09375 96.355227) (end 163.193443 108.255534) (width 0.2) (layer "F.Cu") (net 5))
 (segment (start 163.193443 108.255534) (end 144.143443 108.255534) (width 0.2) (layer "F.Cu") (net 5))
 (segment (start 175.09375 74.009562) (end 175.09375 96.355227) (width 0.2) (layer "F.Cu") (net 5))
 (segment (start 121.44375 73.81875) (end 121.634562 74.009562) (width 0.2) (layer "F.Cu") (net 5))
 (segment (start 124.62142 72.259562) (end 123.825 71.463142) (width 0.2) (layer "F.Cu") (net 17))
 (segment (start 180.975 66.675) (end 180.975 71.628312) (width 0.2) (layer "F.Cu") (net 17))
 (segment (start 123.825 71.463142) (end 123.825 66.675) (width 0.2) (layer "F.Cu") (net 17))
 (segment (start 180.975 71.628312) (end 178.59375 74.009562) (width 0.2) (layer "F.Cu") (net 17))
 (segment (start 123.825 66.675) (end 126.20625 66.675) (width 0.2) (layer "F.Cu") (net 17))
 (via (at 180.975 66.675) (size 0.6) (drill 0.3) (layers "F.Cu" "B.Cu") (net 17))
 (via (at 126.20625 66.675) (size 0.6) (drill 0.3) (layers "F.Cu" "B.Cu") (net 17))
 (segment (start 126.20625 66.675) (end 127.976941 64.904309) (width 0.2) (layer "B.Cu") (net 17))
 (segment (start 127.976941 64.904309) (end 179.204309 64.904309) (width 0.2) (layer "B.Cu") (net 17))
 (segment (start 179.204309 64.904309) (end 180.975 66.675) (width 0.2) (layer "B.Cu") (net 17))
 (segment (start 143.329336 68.507309) (end 141.042691 68.507309) (width 0.2) (layer "F.Cu") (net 10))
 (segment (start 141.042691 68.507309) (end 135.540438 74.009562) (width 0.2) (layer "F.Cu") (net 10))
 (segment (start 135.540438 74.009562) (end 128.12142 74.009562) (width 0.2) (layer "F.Cu") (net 10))
 (segment (start 152.4 76.2) (end 150.01875 78.58125) (width 0.2) (layer "F.Cu") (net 1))
 (segment (start 130.96875 83.307797) (end 131.878971 84.218018) (width 0.2) (layer "F.Cu") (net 1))
 (segment (start 152.4 64.516645) (end 152.4 76.2) (width 0.2) (layer "F.Cu") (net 1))
 (segment (start 150.01875 78.58125) (end 130.96875 78.58125) (width 0.2) (layer "F.Cu") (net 1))
 (segment (start 130.96875 78.58125) (end 130.96875 83.307797) (width 0.2) (layer "F.Cu") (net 1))
 (segment (start 158.569336 58.347309) (end 152.4 64.516645) (width 0.2) (layer "F.Cu") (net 1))
 (segment (start 128.5875 86.006547) (end 128.5875 78.58125) (width 0.2) (layer "F.Cu") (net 3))
 (segment (start 131.878971 89.298018) (end 128.5875 86.006547) (width 0.2) (layer "F.Cu") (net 3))
 (via (at 128.5875 78.58125) (size 0.6) (drill 0.3) (layers "F.Cu" "B.Cu") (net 3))
 (segment (start 141.201441 65.967309) (end 143.329336 65.967309) (width 0.2) (layer "B.Cu") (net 3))
 (segment (start 128.5875 78.58125) (end 141.201441 65.967309) (width 0.2) (layer "B.Cu") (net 3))
 (segment (start 154.78125 64.675395) (end 154.78125 78.58125) (width 0.2) (layer "F.Cu") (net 2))
 (segment (start 154.78125 78.58125) (end 146.604482 86.758018) (width 0.2) (layer "F.Cu") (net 2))
 (segment (start 158.569336 60.887309) (end 154.78125 64.675395) (width 0.2) (layer "F.Cu") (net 2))
 (segment (start 146.604482 86.758018) (end 131.878971 86.758018) (width 0.2) (layer "F.Cu") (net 2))
 (segment (start 150.01875 76.2) (end 126.20625 76.2) (width 0.2) (layer "F.Cu") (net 4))
 (segment (start 123.825 90.4875) (end 126.20625 92.86875) (width 0.2) (layer "F.Cu") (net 4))
 (segment (start 146.771059 63.427309) (end 150.01875 66.675) (width 0.2) (layer "F.Cu") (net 4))
 (segment (start 130.848239 92.86875) (end 131.878971 91.838018) (width 0.2) (layer "F.Cu") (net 4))
 (segment (start 123.825 78.58125) (end 123.825 90.4875) (width 0.2) (layer "F.Cu") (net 4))
 (segment (start 126.20625 76.2) (end 123.825 78.58125) (width 0.2) (layer "F.Cu") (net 4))
 (segment (start 126.20625 92.86875) (end 130.848239 92.86875) (width 0.2) (layer "F.Cu") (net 4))
 (segment (start 150.01875 66.675) (end 150.01875 76.2) (width 0.2) (layer "F.Cu") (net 4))
 (segment (start 143.329336 63.427309) (end 146.771059 63.427309) (width 0.2) (layer "F.Cu") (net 4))
 (segment (start 159.54375 72.021723) (end 159.54375 76.2) (width 0.2) (layer "F.Cu") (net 12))
 (segment (start 158.569336 71.047309) (end 159.54375 72.021723) (width 0.2) (layer "F.Cu") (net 12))
 (via (at 159.54375 76.2) (size 0.6) (drill 0.3) (layers "F.Cu" "B.Cu") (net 12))
 (segment (start 137.793443 97.950307) (end 137.793443 110.795534) (width 0.2) (layer "B.Cu") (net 12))
 (segment (start 159.54375 76.2) (end 137.793443 97.950307) (width 0.2) (layer "B.Cu") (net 12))
 (segment (start 156.843443 110.795534) (end 155.585409 109.5375) (width 0.2) (layer "F.Cu") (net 13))
 (segment (start 155.585409 109.5375) (end 152.4 109.5375) (width 0.2) (layer "F.Cu") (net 13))
 (via (at 152.4 109.5375) (size 0.6) (drill 0.3) (layers "F.Cu" "B.Cu") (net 13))
 (segment (start 161.925 69.05625) (end 159.118277 69.05625) (width 0.2) (layer "B.Cu") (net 13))
 (segment (start 161.925 77.731307) (end 161.925 69.05625) (width 0.2) (layer "B.Cu") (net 13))
 (segment (start 159.118277 69.05625) (end 158.569336 68.507309) (width 0.2) (layer "B.Cu") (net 13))
 (segment (start 152.4 87.256307) (end 161.925 77.731307) (width 0.2) (layer "B.Cu") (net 13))
 (segment (start 152.4 109.5375) (end 152.4 87.256307) (width 0.2) (layer "B.Cu") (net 13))
 (segment (start 158.569336 65.967309) (end 157.506336 67.030309) (width 0.2) (layer "F.Cu") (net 6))
 (segment (start 157.506336 78.925086) (end 159.54375 80.9625) (width 0.2) (layer "F.Cu") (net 6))
 (segment (start 158.569336 65.967309) (end 159.404336 65.967309) (width 0.2) (layer "F.Cu") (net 6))
 (segment (start 157.506336 67.030309) (end 157.506336 78.925086) (width 0.2) (layer "F.Cu") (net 6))
 (via (at 159.54375 80.9625) (size 0.6) (drill 0.3) (layers "F.Cu" "B.Cu") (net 6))
 (segment (start 137.793443 127.86422) (end 137.793443 129.845534) (width 0.2) (layer "B.Cu") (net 6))
 (segment (start 159.54375 80.9625) (end 157.1625 83.34375) (width 0.2) (layer "B.Cu") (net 6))
 (segment (start 157.1625 108.495163) (end 137.793443 127.86422) (width 0.2) (layer "B.Cu") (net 6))
 (segment (start 157.1625 83.34375) (end 157.1625 108.495163) (width 0.2) (layer "B.Cu") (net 6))
 (segment (start 164.30625 66.675) (end 164.30625 80.9625) (width 0.2) (layer "F.Cu") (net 14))
 (segment (start 161.058559 63.427309) (end 164.30625 66.675) (width 0.2) (layer "F.Cu") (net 14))
 (segment (start 158.569336 63.427309) (end 161.058559 63.427309) (width 0.2) (layer "F.Cu") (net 14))
 (via (at 164.30625 80.9625) (size 0.6) (drill 0.3) (layers "F.Cu" "B.Cu") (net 14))
 (segment (start 158.244443 128.444534) (end 156.843443 129.845534) (width 0.2) (layer "B.Cu") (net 14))
 (segment (start 158.244443 87.024307) (end 158.244443 128.444534) (width 0.2) (layer "B.Cu") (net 14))
 (segment (start 164.30625 80.9625) (end 158.244443 87.024307) (width 0.2) (layer "B.Cu") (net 14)))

